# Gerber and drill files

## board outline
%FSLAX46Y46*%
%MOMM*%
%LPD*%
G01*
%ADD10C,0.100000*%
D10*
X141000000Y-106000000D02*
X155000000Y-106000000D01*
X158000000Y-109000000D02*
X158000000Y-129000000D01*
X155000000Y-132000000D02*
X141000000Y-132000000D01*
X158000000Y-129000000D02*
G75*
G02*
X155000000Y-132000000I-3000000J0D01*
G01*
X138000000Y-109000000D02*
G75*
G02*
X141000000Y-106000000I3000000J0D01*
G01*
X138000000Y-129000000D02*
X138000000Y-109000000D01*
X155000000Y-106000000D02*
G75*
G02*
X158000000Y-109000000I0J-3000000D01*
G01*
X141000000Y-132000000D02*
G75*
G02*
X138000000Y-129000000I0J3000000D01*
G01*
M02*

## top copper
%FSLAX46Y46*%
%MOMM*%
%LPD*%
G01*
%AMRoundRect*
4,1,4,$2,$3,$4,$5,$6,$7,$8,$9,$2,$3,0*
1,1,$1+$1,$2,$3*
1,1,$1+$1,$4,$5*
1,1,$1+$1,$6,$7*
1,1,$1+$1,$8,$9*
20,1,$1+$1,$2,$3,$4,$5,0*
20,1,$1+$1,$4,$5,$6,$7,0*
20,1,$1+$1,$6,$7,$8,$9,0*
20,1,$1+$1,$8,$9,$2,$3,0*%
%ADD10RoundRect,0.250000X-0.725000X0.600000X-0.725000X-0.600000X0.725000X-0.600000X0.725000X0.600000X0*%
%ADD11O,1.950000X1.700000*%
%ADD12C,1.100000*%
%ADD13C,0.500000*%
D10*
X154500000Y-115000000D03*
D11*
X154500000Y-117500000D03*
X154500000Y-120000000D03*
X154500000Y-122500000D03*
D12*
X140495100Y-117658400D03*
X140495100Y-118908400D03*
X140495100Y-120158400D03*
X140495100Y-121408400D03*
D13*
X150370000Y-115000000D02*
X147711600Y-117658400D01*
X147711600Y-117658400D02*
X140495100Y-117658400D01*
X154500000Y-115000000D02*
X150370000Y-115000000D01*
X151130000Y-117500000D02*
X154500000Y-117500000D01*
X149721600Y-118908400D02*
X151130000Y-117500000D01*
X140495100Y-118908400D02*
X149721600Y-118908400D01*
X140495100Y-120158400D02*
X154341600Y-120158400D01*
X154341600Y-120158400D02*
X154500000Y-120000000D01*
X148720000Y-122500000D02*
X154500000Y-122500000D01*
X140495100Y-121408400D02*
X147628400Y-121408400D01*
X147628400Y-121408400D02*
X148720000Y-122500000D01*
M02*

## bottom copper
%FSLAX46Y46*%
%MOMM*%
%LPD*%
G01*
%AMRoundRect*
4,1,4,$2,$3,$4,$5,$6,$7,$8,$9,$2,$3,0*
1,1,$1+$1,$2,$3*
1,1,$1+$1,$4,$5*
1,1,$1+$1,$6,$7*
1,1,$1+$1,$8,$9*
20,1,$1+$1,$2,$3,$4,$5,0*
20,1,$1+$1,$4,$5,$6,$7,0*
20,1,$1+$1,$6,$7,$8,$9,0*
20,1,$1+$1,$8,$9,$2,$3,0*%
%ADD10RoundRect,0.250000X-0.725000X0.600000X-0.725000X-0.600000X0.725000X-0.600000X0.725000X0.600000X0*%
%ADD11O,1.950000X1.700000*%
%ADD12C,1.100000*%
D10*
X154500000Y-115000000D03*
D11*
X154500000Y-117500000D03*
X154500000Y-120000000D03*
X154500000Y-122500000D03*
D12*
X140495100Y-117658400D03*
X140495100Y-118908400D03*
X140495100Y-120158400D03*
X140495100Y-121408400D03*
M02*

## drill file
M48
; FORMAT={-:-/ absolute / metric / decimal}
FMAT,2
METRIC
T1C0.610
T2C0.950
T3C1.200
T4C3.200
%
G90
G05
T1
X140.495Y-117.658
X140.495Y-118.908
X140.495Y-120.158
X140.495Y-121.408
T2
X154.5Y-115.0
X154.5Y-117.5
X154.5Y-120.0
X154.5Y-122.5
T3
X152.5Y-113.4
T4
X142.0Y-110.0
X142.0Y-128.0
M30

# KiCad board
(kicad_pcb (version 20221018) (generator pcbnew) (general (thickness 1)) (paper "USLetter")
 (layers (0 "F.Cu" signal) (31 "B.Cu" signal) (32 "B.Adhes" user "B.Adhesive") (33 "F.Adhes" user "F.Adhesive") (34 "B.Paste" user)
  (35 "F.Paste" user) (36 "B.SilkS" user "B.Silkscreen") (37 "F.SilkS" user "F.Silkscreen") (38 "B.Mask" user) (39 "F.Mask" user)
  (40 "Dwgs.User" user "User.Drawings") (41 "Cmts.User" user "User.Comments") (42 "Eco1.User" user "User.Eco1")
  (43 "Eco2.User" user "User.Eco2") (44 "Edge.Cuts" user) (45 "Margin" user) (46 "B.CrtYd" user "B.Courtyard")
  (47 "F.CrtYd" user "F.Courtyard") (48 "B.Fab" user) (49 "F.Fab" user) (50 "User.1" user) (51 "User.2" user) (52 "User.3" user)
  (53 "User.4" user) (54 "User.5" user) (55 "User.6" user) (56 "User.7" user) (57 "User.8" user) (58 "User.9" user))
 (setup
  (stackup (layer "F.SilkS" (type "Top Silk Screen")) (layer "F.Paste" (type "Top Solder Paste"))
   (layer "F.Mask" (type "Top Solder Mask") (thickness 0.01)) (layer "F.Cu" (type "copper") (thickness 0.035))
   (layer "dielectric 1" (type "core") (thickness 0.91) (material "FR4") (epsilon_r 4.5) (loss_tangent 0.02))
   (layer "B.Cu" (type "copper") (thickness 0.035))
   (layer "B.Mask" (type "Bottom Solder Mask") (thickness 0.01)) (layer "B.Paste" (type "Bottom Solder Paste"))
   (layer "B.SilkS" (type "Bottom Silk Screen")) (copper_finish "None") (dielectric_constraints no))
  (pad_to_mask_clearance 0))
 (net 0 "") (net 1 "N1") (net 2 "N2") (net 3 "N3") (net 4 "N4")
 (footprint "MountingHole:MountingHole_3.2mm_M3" (layer "F.Cu") (at 142 110)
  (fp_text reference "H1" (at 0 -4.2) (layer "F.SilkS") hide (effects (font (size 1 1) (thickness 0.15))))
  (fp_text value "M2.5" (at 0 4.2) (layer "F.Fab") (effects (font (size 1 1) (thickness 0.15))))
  (pad "" np_thru_hole circle (at 0 0) (size 3.2 3.2) (drill 3.2) (layers "*.Cu" "*.Mask")))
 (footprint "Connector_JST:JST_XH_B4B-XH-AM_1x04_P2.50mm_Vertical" (layer "F.Cu") (at 154.5 115 -90)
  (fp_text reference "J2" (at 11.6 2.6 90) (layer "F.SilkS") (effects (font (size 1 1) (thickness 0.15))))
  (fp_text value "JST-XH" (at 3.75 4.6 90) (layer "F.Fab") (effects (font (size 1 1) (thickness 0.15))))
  (pad "" np_thru_hole circle (at -1.6 2 270) (size 1.2 1.2) (drill 1.2) (layers "*.Cu" "*.Mask"))
  (pad "1" thru_hole roundrect (at 0 0 270) (size 1.7 1.95) (drill 0.95) (layers "*.Cu" "*.Mask") (roundrect_rratio 0.1470588235)
   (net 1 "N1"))
  (pad "2" thru_hole oval (at 2.5 0 270) (size 1.7 1.95) (drill 0.95) (layers "*.Cu" "*.Mask") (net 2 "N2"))
  (pad "3" thru_hole oval (at 5 0 270) (size 1.7 1.95) (drill 0.95) (layers "*.Cu" "*.Mask") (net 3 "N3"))
  (pad "4" thru_hole oval (at 7.5 0 270) (size 1.7 1.95) (drill 0.95) (layers "*.Cu" "*.Mask") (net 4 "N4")))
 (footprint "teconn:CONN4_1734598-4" (layer "F.Cu") (at 140.4951 117.6584 90)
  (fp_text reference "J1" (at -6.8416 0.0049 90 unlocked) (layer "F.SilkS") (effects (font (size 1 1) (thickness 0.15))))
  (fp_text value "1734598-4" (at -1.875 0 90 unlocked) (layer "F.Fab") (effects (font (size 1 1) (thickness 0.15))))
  (pad "1" thru_hole circle (at 0 0 90) (size 1.1 1.1) (drill 0.6096) (layers "*.Cu" "*.Mask") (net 1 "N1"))
  (pad "2" thru_hole circle (at -1.25 0 90) (size 1.1 1.1) (drill 0.6096) (layers "*.Cu" "*.Mask") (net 2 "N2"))
  (pad "3" thru_hole circle (at -2.5 0 90) (size 1.1 1.1) (drill 0.6096) (layers "*.Cu" "*.Mask") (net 3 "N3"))
  (pad "4" thru_hole circle (at -3.75 0 90) (size 1.1 1.1) (drill 0.6096) (layers "*.Cu" "*.Mask") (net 4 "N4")))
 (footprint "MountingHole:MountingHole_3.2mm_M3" (layer "F.Cu") (at 142 128)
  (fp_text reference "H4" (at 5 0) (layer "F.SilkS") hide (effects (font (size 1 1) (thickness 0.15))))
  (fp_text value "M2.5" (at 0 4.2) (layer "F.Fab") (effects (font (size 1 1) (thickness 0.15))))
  (pad "" np_thru_hole circle (at 0 0) (size 3.2 3.2) (drill 3.2) (layers "*.Cu" "*.Mask")))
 (gr_line (start 141 106) (end 155 106) (stroke (width 0.1) (type default)) (layer "Edge.Cuts"))
 (gr_line (start 158 109) (end 158 129) (stroke (width 0.1) (type default)) (layer "Edge.Cuts"))
 (gr_line (start 155 132) (end 141 132) (stroke (width 0.1) (type default)) (layer "Edge.Cuts"))
 (gr_arc (start 158 129) (mid 157.12132 131.12132) (end 155 132) (stroke (width 0.1) (type default)) (layer "Edge.Cuts"))
 (gr_arc (start 138 109) (mid 138.87868 106.87868) (end 141 106) (stroke (width 0.1) (type default)) (layer "Edge.Cuts"))
 (gr_line (start 138 129) (end 138 109) (stroke (width 0.1) (type default)) (layer "Edge.Cuts"))
 (gr_arc (start 155 106) (mid 157.12132 106.87868) (end 158 109) (stroke (width 0.1) (type default)) (layer "Edge.Cuts"))
 (gr_arc (start 141 132) (mid 138.87868 131.12132) (end 138 129) (stroke (width 0.1) (type default)) (layer "Edge.Cuts"))
 (segment (start 150.37 115) (end 147.7116 117.6584) (width 0.5) (layer "F.Cu") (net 1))
 (segment (start 147.7116 117.6584) (end 140.4951 117.6584) (width 0.5) (layer "F.Cu") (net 1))
 (segment (start 154.5 115) (end 150.37 115) (width 0.5) (layer "F.Cu") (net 1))
 (segment (start 151.13 117.5) (end 154.5 117.5) (width 0.5) (layer "F.Cu") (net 2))
 (segment (start 149.7216 118.9084) (end 151.13 117.5) (width 0.5) (layer "F.Cu") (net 2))
 (segment (start 140.4951 118.9084) (end 149.7216 118.9084) (width 0.5) (layer "F.Cu") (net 2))
 (segment (start 140.4951 120.1584) (end 154.3416 120.1584) (width 0.5) (layer "F.Cu") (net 3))
 (segment (start 154.3416 120.1584) (end 154.5 120) (width 0.5) (layer "F.Cu") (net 3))
 (segment (start 148.72 122.5) (end 154.5 122.5) (width 0.5) (layer "F.Cu") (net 4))
 (segment (start 140.4951 121.4084) (end 147.6284 121.4084) (width 0.5) (layer "F.Cu") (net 4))
 (segment (start 147.6284 121.4084) (end 148.72 122.5) (width 0.5) (layer "F.Cu") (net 4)))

